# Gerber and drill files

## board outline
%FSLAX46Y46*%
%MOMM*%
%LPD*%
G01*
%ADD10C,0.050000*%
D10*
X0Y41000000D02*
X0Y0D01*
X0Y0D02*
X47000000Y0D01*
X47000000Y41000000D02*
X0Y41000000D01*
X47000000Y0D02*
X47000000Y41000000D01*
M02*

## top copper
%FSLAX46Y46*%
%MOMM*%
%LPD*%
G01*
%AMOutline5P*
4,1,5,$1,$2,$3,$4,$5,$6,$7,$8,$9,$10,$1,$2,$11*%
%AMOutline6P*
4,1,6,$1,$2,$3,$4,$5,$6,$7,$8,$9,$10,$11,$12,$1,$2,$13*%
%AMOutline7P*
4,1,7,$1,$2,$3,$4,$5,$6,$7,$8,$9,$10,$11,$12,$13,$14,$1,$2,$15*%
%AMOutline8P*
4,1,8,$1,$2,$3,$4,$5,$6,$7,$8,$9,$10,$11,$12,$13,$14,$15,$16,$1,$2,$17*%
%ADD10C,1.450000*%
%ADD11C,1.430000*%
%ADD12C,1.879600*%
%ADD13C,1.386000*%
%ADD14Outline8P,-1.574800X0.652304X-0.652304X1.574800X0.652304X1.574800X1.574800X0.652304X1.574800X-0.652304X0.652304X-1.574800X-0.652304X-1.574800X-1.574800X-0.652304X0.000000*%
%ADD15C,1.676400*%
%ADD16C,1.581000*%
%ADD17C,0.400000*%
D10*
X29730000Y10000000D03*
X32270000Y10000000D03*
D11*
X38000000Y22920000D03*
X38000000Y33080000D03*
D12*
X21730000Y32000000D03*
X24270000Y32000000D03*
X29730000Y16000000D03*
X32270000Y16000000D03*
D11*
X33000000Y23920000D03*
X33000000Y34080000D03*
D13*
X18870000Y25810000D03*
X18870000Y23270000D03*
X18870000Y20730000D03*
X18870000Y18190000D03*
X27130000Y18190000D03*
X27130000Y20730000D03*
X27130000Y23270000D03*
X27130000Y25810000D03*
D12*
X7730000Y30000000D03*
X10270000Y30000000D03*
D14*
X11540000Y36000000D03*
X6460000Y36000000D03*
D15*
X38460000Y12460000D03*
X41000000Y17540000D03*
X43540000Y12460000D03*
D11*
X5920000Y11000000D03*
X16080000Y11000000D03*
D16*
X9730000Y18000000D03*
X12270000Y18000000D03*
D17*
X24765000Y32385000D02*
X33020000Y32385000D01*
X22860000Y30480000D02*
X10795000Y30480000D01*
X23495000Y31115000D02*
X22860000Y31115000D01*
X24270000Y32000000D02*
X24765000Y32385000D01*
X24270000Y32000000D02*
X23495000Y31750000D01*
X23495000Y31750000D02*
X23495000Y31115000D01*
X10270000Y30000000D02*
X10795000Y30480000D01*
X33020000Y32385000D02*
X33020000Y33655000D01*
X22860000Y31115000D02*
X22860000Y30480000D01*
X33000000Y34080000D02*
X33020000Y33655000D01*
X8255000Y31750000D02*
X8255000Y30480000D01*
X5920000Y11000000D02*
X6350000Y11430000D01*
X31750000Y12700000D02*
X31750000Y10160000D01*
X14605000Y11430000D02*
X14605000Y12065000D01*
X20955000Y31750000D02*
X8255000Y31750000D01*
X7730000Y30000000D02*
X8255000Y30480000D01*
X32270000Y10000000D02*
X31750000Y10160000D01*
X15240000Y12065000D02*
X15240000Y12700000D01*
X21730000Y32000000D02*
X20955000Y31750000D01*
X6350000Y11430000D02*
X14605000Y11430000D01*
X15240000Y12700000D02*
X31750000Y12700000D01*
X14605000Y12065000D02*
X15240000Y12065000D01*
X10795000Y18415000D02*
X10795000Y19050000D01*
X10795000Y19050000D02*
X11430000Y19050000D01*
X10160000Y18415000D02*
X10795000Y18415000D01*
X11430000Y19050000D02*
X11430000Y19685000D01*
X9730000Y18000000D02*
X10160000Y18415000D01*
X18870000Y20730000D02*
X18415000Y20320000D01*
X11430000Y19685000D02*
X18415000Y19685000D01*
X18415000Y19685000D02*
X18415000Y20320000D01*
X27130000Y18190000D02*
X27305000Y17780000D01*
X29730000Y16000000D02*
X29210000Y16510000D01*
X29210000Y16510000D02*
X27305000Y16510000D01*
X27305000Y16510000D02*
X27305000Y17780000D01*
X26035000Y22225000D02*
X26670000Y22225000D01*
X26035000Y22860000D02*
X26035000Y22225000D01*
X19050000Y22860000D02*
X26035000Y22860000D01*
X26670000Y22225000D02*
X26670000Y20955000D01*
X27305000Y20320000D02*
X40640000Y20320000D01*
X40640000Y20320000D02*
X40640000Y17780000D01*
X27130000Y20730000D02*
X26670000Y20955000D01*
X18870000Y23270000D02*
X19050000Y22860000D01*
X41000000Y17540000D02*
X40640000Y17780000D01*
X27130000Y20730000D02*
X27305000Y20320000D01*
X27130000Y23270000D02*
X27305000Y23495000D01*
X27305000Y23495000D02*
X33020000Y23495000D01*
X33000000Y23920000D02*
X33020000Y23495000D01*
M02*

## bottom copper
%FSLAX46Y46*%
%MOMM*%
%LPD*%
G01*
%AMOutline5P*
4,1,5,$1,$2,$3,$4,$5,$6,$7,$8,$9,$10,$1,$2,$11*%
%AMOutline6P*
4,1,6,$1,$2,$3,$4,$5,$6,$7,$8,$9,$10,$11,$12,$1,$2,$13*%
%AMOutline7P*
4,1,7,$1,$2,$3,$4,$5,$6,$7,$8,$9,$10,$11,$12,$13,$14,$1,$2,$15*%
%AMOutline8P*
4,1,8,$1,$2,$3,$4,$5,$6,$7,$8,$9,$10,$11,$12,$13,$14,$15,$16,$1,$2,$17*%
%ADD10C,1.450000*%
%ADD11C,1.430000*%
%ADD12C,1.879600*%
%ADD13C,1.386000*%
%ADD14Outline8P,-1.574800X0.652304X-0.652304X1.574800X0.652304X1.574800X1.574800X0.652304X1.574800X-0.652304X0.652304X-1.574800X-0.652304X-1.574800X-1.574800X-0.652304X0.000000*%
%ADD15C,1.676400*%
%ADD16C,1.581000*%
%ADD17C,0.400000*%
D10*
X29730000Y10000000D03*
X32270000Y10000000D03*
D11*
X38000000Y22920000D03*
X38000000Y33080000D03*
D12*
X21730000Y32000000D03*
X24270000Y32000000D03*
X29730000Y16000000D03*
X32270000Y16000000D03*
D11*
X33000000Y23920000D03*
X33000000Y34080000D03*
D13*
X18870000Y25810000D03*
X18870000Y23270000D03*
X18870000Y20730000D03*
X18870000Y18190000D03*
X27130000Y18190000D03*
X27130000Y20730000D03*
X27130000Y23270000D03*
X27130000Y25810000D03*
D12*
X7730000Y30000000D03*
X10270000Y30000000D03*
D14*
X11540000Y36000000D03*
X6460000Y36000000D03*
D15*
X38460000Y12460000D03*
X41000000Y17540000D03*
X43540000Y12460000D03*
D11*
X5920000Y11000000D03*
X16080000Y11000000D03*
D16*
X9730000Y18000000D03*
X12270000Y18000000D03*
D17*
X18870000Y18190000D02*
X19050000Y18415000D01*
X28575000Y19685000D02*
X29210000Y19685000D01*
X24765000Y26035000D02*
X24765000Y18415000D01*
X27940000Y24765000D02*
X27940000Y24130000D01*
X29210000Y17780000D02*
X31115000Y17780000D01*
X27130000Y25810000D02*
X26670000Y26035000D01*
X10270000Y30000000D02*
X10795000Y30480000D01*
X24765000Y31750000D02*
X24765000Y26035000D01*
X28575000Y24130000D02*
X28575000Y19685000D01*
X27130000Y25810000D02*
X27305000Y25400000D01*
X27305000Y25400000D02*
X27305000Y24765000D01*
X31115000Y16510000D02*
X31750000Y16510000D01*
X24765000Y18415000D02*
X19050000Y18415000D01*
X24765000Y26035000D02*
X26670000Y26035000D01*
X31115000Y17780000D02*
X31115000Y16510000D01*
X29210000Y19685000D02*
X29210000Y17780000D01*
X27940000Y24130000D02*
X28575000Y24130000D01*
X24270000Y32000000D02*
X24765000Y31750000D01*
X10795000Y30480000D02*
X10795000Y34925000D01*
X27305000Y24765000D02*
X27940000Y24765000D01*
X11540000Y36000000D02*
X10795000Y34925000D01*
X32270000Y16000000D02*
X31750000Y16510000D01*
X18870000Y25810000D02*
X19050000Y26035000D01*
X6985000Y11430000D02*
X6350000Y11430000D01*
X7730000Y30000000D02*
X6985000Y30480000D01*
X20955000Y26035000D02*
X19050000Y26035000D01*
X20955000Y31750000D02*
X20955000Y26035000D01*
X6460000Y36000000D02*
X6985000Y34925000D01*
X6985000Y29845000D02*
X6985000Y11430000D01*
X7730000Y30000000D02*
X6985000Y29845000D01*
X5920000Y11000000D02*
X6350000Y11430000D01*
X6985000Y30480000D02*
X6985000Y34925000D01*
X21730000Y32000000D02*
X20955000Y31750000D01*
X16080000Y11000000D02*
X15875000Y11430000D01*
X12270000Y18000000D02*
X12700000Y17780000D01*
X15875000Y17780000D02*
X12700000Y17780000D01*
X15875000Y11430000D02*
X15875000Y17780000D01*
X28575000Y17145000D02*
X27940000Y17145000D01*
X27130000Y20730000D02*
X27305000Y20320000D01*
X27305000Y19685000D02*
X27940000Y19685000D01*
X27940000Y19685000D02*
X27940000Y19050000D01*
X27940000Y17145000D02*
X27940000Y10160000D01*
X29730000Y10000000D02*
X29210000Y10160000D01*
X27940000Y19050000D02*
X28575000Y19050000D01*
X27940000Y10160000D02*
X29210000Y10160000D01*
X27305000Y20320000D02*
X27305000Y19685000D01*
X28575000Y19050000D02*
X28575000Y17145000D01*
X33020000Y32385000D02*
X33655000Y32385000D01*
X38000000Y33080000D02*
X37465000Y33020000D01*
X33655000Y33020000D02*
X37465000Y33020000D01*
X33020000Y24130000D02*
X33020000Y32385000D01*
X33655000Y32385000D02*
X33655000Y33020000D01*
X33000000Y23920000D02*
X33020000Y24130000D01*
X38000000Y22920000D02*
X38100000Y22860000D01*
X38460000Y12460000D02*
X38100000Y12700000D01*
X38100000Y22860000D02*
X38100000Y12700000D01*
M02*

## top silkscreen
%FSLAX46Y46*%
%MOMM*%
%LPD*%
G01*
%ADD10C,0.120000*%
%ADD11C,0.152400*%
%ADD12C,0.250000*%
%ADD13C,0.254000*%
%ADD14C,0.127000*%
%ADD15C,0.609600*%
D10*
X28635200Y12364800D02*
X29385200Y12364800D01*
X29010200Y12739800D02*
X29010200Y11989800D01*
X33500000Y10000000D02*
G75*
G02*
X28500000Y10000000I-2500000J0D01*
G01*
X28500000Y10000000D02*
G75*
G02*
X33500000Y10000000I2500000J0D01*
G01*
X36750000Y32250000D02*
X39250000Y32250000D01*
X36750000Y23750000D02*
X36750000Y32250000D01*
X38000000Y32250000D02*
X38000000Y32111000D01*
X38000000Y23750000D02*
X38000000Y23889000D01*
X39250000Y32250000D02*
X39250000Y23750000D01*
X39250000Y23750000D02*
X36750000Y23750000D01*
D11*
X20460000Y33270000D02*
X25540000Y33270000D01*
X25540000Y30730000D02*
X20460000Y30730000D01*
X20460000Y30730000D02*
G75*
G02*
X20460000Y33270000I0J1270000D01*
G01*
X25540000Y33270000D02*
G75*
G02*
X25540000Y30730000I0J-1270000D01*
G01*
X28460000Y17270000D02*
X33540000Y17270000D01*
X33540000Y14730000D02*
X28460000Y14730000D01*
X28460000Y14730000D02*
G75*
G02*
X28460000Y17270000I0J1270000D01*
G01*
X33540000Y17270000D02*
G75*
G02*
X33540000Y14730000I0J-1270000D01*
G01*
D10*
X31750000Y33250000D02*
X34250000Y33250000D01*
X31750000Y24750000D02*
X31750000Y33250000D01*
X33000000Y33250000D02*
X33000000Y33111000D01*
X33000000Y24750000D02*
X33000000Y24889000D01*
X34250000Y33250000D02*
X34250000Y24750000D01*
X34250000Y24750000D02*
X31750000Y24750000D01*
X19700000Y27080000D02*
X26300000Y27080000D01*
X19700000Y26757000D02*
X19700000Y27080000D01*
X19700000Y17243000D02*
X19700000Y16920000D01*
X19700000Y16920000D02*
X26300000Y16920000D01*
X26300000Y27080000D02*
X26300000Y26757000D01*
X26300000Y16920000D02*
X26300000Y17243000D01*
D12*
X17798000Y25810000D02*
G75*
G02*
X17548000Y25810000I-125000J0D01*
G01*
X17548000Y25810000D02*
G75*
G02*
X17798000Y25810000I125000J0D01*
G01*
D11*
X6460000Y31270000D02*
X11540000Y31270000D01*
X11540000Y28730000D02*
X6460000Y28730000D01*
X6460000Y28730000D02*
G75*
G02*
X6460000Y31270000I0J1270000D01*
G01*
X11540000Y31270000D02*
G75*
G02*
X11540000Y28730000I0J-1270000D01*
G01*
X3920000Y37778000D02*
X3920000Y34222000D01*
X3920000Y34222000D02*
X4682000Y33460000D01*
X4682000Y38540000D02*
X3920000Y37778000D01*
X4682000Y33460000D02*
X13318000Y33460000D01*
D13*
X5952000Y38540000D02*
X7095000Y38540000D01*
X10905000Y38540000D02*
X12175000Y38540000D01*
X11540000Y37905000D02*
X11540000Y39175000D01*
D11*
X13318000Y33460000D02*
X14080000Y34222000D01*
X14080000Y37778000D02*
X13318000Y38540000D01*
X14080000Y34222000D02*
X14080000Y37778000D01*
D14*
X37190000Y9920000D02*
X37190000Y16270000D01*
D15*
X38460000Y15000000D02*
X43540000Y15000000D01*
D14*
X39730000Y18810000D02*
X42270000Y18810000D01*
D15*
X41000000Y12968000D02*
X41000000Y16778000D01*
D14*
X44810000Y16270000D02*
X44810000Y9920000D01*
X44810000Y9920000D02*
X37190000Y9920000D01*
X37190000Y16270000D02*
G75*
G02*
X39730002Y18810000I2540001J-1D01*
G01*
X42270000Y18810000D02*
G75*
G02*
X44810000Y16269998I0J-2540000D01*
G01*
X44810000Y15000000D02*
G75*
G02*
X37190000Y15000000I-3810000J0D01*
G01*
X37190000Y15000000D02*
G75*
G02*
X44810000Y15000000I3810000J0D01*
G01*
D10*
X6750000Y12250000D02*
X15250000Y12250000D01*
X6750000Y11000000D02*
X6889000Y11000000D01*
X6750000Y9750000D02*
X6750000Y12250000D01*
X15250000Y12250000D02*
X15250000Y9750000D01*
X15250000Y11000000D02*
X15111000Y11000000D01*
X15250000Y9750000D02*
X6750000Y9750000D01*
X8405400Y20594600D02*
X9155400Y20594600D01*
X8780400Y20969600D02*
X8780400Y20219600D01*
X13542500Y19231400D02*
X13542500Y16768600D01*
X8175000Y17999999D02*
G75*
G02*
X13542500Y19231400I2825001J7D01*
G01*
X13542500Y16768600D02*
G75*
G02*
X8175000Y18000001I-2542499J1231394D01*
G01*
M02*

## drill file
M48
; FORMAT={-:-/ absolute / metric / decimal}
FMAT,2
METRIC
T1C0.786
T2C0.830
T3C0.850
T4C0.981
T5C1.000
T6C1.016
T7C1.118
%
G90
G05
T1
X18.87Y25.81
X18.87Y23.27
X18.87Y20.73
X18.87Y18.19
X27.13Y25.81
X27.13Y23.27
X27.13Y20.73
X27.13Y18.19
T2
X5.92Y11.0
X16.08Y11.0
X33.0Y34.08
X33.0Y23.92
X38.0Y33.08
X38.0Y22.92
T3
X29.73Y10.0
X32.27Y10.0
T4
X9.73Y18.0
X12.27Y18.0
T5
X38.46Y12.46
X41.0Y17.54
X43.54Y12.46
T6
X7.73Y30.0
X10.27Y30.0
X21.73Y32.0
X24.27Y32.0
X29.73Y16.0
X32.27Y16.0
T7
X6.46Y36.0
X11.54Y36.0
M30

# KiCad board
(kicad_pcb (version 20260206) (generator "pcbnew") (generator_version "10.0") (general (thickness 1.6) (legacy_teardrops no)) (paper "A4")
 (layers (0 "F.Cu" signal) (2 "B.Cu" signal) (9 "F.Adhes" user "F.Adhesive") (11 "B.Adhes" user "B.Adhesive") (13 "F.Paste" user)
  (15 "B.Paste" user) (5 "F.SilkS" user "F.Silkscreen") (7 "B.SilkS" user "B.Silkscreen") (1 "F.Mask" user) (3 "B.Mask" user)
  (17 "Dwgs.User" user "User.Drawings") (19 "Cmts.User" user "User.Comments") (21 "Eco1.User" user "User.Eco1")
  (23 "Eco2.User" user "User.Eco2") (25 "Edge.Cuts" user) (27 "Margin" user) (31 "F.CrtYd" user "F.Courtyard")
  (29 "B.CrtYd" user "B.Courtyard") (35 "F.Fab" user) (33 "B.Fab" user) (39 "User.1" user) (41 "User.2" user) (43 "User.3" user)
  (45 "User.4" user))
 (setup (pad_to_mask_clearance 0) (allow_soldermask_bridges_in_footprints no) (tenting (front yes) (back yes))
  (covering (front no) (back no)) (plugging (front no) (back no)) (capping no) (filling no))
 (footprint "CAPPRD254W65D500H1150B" (layer "F.Cu") (at 31 -10)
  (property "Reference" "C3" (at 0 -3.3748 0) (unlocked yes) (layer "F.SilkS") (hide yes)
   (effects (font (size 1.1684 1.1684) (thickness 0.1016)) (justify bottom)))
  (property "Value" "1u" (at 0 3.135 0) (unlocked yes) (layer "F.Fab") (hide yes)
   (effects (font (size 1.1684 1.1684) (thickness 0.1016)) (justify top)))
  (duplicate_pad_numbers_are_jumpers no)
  (fp_line (start -2.3648 -2.3648) (end -1.6148 -2.3648) (stroke (width 0.12) (type solid)) (layer "F.SilkS"))
  (fp_line (start -1.9898 -2.7398) (end -1.9898 -1.9898) (stroke (width 0.12) (type solid)) (layer "F.SilkS"))
  (fp_circle (center 0 0) (end 2.5 0) (stroke (width 0.12) (type solid)) (fill no) (layer "F.SilkS"))
  (pad "1" thru_hole circle (at -1.27 0) (size 1.45 1.45) (drill 0.85) (layers "*.Cu" "*.Mask") (remove_unused_layers no) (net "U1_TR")
   (solder_mask_margin 0.1016) (thermal_bridge_angle 0))
  (pad "2" thru_hole circle (at 1.27 0) (size 1.45 1.45) (drill 0.85) (layers "*.Cu" "*.Mask") (remove_unused_layers no) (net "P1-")
   (solder_mask_margin 0.1016) (thermal_bridge_angle 0)))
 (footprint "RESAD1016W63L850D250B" (layer "F.Cu") (at 38 -28 90)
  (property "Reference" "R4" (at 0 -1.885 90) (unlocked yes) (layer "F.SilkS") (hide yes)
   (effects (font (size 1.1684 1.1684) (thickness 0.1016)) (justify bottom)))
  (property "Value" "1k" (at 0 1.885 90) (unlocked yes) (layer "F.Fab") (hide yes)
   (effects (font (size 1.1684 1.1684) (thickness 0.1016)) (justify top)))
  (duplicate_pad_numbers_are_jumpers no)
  (fp_line (start 4.25 -1.25) (end 4.25 1.25) (stroke (width 0.12) (type solid)) (layer "F.SilkS"))
  (fp_line (start -4.25 -1.25) (end 4.25 -1.25) (stroke (width 0.12) (type solid)) (layer "F.SilkS"))
  (fp_line (start 4.25 0) (end 4.111 0) (stroke (width 0.12) (type solid)) (layer "F.SilkS"))
  (fp_line (start -4.25 0) (end -4.111 0) (stroke (width 0.12) (type solid)) (layer "F.SilkS"))
  (fp_line (start 4.25 1.25) (end -4.25 1.25) (stroke (width 0.12) (type solid)) (layer "F.SilkS"))
  (fp_line (start -4.25 1.25) (end -4.25 -1.25) (stroke (width 0.12) (type solid)) (layer "F.SilkS"))
  (pad "1" thru_hole circle (at -5.08 0 90) (size 1.43 1.43) (drill 0.83) (layers "*.Cu" "*.Mask") (remove_unused_layers no)
   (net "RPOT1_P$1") (solder_mask_margin 0.1016) (thermal_bridge_angle 0))
  (pad "2" thru_hole circle (at 5.08 0 90) (size 1.43 1.43) (drill 0.83) (layers "*.Cu" "*.Mask") (remove_unused_layers no) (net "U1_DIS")
   (solder_mask_margin 0.1016) (thermal_bridge_angle 0)))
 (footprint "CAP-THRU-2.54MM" (layer "F.Cu") (at 23 -32)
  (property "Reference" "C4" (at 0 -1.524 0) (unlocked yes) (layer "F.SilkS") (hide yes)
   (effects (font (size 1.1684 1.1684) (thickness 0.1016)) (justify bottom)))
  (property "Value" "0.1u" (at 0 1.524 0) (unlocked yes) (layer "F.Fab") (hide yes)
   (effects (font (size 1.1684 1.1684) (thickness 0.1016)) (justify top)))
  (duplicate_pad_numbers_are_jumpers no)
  (fp_line (start -2.54 -1.27) (end 2.54 -1.27) (stroke (width 0.1524) (type solid)) (layer "F.SilkS"))
  (fp_line (start 2.54 1.27) (end -2.54 1.27) (stroke (width 0.1524) (type solid)) (layer "F.SilkS"))
  (fp_arc (start -2.54 1.27) (mid -3.81 0) (end -2.54 -1.27) (stroke (width 0.1524) (type solid)) (layer "F.SilkS"))
  (fp_arc (start 2.54 -1.27) (mid 3.81 0) (end 2.54 1.27) (stroke (width 0.1524) (type solid)) (layer "F.SilkS"))
  (pad "1" thru_hole circle (at -1.27 0) (size 1.8796 1.8796) (drill 1.016) (layers "*.Cu" "*.Mask") (remove_unused_layers no) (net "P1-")
   (solder_mask_margin 0.1016) (thermal_bridge_angle 0))
  (pad "2" thru_hole circle (at 1.27 0) (size 1.8796 1.8796) (drill 1.016) (layers "*.Cu" "*.Mask") (remove_unused_layers no) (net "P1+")
   (solder_mask_margin 0.1016) (thermal_bridge_angle 0)))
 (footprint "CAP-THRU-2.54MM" (layer "F.Cu") (at 31 -16)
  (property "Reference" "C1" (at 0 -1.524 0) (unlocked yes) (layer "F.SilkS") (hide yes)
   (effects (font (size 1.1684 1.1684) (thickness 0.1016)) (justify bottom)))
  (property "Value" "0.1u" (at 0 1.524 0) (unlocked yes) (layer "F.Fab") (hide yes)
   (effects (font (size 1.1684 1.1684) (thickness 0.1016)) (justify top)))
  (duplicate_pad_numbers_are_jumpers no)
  (fp_line (start -2.54 -1.27) (end 2.54 -1.27) (stroke (width 0.1524) (type solid)) (layer "F.SilkS"))
  (fp_line (start 2.54 1.27) (end -2.54 1.27) (stroke (width 0.1524) (type solid)) (layer "F.SilkS"))
  (fp_arc (start -2.54 1.27) (mid -3.81 0) (end -2.54 -1.27) (stroke (width 0.1524) (type solid)) (layer "F.SilkS"))
  (fp_arc (start 2.54 -1.27) (mid 3.81 0) (end 2.54 1.27) (stroke (width 0.1524) (type solid)) (layer "F.SilkS"))
  (pad "1" thru_hole circle (at -1.27 0) (size 1.8796 1.8796) (drill 1.016) (layers "*.Cu" "*.Mask") (remove_unused_layers no) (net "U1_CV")
   (solder_mask_margin 0.1016) (thermal_bridge_angle 0))
  (pad "2" thru_hole circle (at 1.27 0) (size 1.8796 1.8796) (drill 1.016) (layers "*.Cu" "*.Mask") (remove_unused_layers no) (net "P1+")
   (solder_mask_margin 0.1016) (thermal_bridge_angle 0)))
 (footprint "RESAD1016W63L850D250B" (layer "F.Cu") (at 33 -29 90)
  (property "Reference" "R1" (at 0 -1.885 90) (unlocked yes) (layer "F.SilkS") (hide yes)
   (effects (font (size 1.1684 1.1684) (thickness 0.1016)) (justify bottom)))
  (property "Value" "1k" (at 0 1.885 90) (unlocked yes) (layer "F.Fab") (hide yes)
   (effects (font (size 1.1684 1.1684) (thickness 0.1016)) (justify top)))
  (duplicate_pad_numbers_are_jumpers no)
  (fp_line (start 4.25 -1.25) (end 4.25 1.25) (stroke (width 0.12) (type solid)) (layer "F.SilkS"))
  (fp_line (start -4.25 -1.25) (end 4.25 -1.25) (stroke (width 0.12) (type solid)) (layer "F.SilkS"))
  (fp_line (start 4.25 0) (end 4.111 0) (stroke (width 0.12) (type solid)) (layer "F.SilkS"))
  (fp_line (start -4.25 0) (end -4.111 0) (stroke (width 0.12) (type solid)) (layer "F.SilkS"))
  (fp_line (start 4.25 1.25) (end -4.25 1.25) (stroke (width 0.12) (type solid)) (layer "F.SilkS"))
  (fp_line (start -4.25 1.25) (end -4.25 -1.25) (stroke (width 0.12) (type solid)) (layer "F.SilkS"))
  (pad "1" thru_hole circle (at -5.08 0 90) (size 1.43 1.43) (drill 0.83) (layers "*.Cu" "*.Mask") (remove_unused_layers no) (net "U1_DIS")
   (solder_mask_margin 0.1016) (thermal_bridge_angle 0))
  (pad "2" thru_hole circle (at 5.08 0 90) (size 1.43 1.43) (drill 0.83) (layers "*.Cu" "*.Mask") (remove_unused_layers no) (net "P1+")
   (solder_mask_margin 0.1016) (thermal_bridge_angle 0)))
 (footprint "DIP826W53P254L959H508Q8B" (layer "F.Cu") (at 23 -22)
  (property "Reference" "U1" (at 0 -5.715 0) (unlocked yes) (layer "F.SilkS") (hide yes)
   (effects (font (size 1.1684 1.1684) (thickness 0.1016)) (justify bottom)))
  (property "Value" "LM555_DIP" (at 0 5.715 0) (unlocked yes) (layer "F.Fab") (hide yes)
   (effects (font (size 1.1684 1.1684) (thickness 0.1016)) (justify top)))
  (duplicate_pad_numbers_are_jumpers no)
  (fp_line (start -3.3 -5.08) (end 3.3 -5.08) (stroke (width 0.12) (type solid)) (layer "F.SilkS"))
  (fp_line (start -3.3 -4.757) (end -3.3 -5.08) (stroke (width 0.12) (type solid)) (layer "F.SilkS"))
  (fp_line (start -3.3 4.757) (end -3.3 5.08) (stroke (width 0.12) (type solid)) (layer "F.SilkS"))
  (fp_line (start -3.3 5.08) (end 3.3 5.08) (stroke (width 0.12) (type solid)) (layer "F.SilkS"))
  (fp_line (start 3.3 -5.08) (end 3.3 -4.757) (stroke (width 0.12) (type solid)) (layer "F.SilkS"))
  (fp_line (start 3.3 5.08) (end 3.3 4.757) (stroke (width 0.12) (type solid)) (layer "F.SilkS"))
  (fp_circle (center -5.327 -3.81) (end -5.202 -3.81) (stroke (width 0.25) (type solid)) (fill yes) (layer "F.SilkS"))
  (pad "1" thru_hole circle (at -4.13 -3.81) (size 1.386 1.386) (drill 0.786) (layers "*.Cu" "*.Mask") (remove_unused_layers no) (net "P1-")
   (solder_mask_margin 0.1016) (thermal_bridge_angle 0))
  (pad "2" thru_hole circle (at -4.13 -1.27) (size 1.386 1.386) (drill 0.786) (layers "*.Cu" "*.Mask") (remove_unused_layers no)
   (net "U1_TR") (solder_mask_margin 0.1016) (thermal_bridge_angle 0))
  (pad "3" thru_hole circle (at -4.13 1.27) (size 1.386 1.386) (drill 0.786) (layers "*.Cu" "*.Mask") (remove_unused_layers no)
   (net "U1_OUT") (solder_mask_margin 0.1016) (thermal_bridge_angle 0))
  (pad "4" thru_hole circle (at -4.13 3.81) (size 1.386 1.386) (drill 0.786) (layers "*.Cu" "*.Mask") (remove_unused_layers no) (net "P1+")
   (solder_mask_margin 0.1016) (thermal_bridge_angle 0))
  (pad "5" thru_hole circle (at 4.13 3.81) (size 1.386 1.386) (drill 0.786) (layers "*.Cu" "*.Mask") (remove_unused_layers no) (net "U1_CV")
   (solder_mask_margin 0.1016) (thermal_bridge_angle 0))
  (pad "6" thru_hole circle (at 4.13 1.27) (size 1.386 1.386) (drill 0.786) (layers "*.Cu" "*.Mask") (remove_unused_layers no) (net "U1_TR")
   (solder_mask_margin 0.1016) (thermal_bridge_angle 0))
  (pad "7" thru_hole circle (at 4.13 -1.27) (size 1.386 1.386) (drill 0.786) (layers "*.Cu" "*.Mask") (remove_unused_layers no)
   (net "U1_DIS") (solder_mask_margin 0.1016) (thermal_bridge_angle 0))
  (pad "8" thru_hole circle (at 4.13 -3.81) (size 1.386 1.386) (drill 0.786) (layers "*.Cu" "*.Mask") (remove_unused_layers no) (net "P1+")
   (solder_mask_margin 0.1016) (thermal_bridge_angle 0)))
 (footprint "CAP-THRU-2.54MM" (layer "F.Cu") (at 9 -30)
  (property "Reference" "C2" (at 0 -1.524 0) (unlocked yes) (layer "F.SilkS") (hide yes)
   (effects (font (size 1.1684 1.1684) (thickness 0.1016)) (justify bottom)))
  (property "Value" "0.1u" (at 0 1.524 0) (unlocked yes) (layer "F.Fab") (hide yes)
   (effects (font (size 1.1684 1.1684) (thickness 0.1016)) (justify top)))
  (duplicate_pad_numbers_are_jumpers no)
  (fp_line (start -2.54 -1.27) (end 2.54 -1.27) (stroke (width 0.1524) (type solid)) (layer "F.SilkS"))
  (fp_line (start 2.54 1.27) (end -2.54 1.27) (stroke (width 0.1524) (type solid)) (layer "F.SilkS"))
  (fp_arc (start -2.54 1.27) (mid -3.81 0) (end -2.54 -1.27) (stroke (width 0.1524) (type solid)) (layer "F.SilkS"))
  (fp_arc (start 2.54 -1.27) (mid 3.81 0) (end 2.54 1.27) (stroke (width 0.1524) (type solid)) (layer "F.SilkS"))
  (pad "1" thru_hole circle (at -1.27 0) (size 1.8796 1.8796) (drill 1.016) (layers "*.Cu" "*.Mask") (remove_unused_layers no) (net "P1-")
   (solder_mask_margin 0.1016) (thermal_bridge_angle 0))
  (pad "2" thru_hole circle (at 1.27 0) (size 1.8796 1.8796) (drill 1.016) (layers "*.Cu" "*.Mask") (remove_unused_layers no) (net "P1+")
   (solder_mask_margin 0.1016) (thermal_bridge_angle 0)))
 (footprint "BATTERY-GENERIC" (layer "F.Cu") (at 9 -36)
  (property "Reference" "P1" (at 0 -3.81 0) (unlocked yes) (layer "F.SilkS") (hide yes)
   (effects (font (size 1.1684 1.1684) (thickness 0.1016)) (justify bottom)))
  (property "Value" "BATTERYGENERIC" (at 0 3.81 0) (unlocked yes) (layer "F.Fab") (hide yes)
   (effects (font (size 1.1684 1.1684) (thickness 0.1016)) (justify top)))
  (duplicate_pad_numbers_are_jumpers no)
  (fp_line (start -5.08 -1.778) (end -5.08 1.778) (stroke (width 0.1524) (type solid)) (layer "F.SilkS"))
  (fp_line (start -5.08 1.778) (end -4.318 2.54) (stroke (width 0.1524) (type solid)) (layer "F.SilkS"))
  (fp_line (start -4.318 -2.54) (end -5.08 -1.778) (stroke (width 0.1524) (type solid)) (layer "F.SilkS"))
  (fp_line (start -4.318 2.54) (end 4.318 2.54) (stroke (width 0.1524) (type solid)) (layer "F.SilkS"))
  (fp_line (start -3.048 -2.54) (end -1.905 -2.54) (stroke (width 0.254) (type solid)) (layer "F.SilkS"))
  (fp_line (start 1.905 -2.54) (end 3.175 -2.54) (stroke (width 0.254) (type solid)) (layer "F.SilkS"))
  (fp_line (start 2.54 -1.905) (end 2.54 -3.175) (stroke (width 0.254) (type solid)) (layer "F.SilkS"))
  (fp_line (start 4.318 2.54) (end 5.08 1.778) (stroke (width 0.1524) (type solid)) (layer "F.SilkS"))
  (fp_line (start 5.08 -1.778) (end 4.318 -2.54) (stroke (width 0.1524) (type solid)) (layer "F.SilkS"))
  (fp_line (start 5.08 1.778) (end 5.08 -1.778) (stroke (width 0.1524) (type solid)) (layer "F.SilkS"))
  (pad "+" thru_hole roundrect (at 2.54 0) (size 3.1496 3.1496) (drill 1.1176) (layers "*.Cu" "*.Mask") (remove_unused_layers no)
   (roundrect_rratio 0.25) (chamfer_ratio 0.2928932188) (chamfer top_left top_right bottom_left bottom_right) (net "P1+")
   (solder_mask_margin 0.1016) (thermal_bridge_angle 0))
  (pad "-" thru_hole roundrect (at -2.54 0) (size 3.1496 3.1496) (drill 1.1176) (layers "*.Cu" "*.Mask") (remove_unused_layers no)
   (roundrect_rratio 0.25) (chamfer_ratio 0.2928932188) (chamfer top_left top_right bottom_left bottom_right) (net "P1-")
   (solder_mask_margin 0.1016) (thermal_bridge_angle 0)))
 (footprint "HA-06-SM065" (layer "F.Cu") (at 41 -15)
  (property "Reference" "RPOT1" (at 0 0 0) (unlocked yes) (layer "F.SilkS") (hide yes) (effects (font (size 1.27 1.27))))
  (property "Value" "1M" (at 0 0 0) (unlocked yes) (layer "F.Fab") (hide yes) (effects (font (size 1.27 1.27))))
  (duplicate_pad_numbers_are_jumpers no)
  (fp_line (start -3.81 5.08) (end -3.81 -1.27) (stroke (width 0.127) (type solid)) (layer "F.SilkS"))
  (fp_line (start -2.54 0) (end 2.54 0) (stroke (width 0.6096) (type solid)) (layer "F.SilkS"))
  (fp_line (start -1.27 -3.81) (end 1.27 -3.81) (stroke (width 0.127) (type solid)) (layer "F.SilkS"))
  (fp_line (start 0 2.032) (end 0 -1.778) (stroke (width 0.6096) (type solid)) (layer "F.SilkS"))
  (fp_line (start 3.81 -1.27) (end 3.81 5.08) (stroke (width 0.127) (type solid)) (layer "F.SilkS"))
  (fp_line (start 3.81 5.08) (end -3.81 5.08) (stroke (width 0.127) (type solid)) (layer "F.SilkS"))
  (fp_arc (start -3.81 -1.27) (mid -3.06605 -3.066052) (end -1.269998 -3.81) (stroke (width 0.127) (type solid)) (layer "F.SilkS"))
  (fp_arc (start 1.27 -3.81) (mid 3.066052 -3.06605) (end 3.81 -1.269998) (stroke (width 0.127) (type solid)) (layer "F.SilkS"))
  (fp_circle (center 0 0) (end 3.81 0) (stroke (width 0.127) (type solid)) (fill no) (layer "F.SilkS"))
  (pad "1" thru_hole circle (at -2.54 2.54) (size 1.6764 1.6764) (drill 1) (layers "*.Cu" "*.Mask") (remove_unused_layers no)
   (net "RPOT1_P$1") (solder_mask_margin 0.1016) (thermal_bridge_angle 0))
  (pad "2" thru_hole circle (at 0 -2.54) (size 1.6764 1.6764) (drill 1) (layers "*.Cu" "*.Mask") (remove_unused_layers no) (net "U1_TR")
   (solder_mask_margin 0.1016) (thermal_bridge_angle 0))
  (pad "3" thru_hole circle (at 2.54 2.54) (size 1.6764 1.6764) (drill 1) (layers "*.Cu" "*.Mask") (remove_unused_layers no)
   (solder_mask_margin 0.1016) (thermal_bridge_angle 0)))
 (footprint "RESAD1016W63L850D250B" (layer "F.Cu") (at 11 -11)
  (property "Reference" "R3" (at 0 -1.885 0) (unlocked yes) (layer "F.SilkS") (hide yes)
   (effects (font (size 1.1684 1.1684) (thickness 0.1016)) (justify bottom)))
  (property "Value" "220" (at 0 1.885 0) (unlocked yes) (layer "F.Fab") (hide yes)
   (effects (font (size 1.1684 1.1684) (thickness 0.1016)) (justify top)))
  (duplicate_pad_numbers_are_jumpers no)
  (fp_line (start -4.25 -1.25) (end 4.25 -1.25) (stroke (width 0.12) (type solid)) (layer "F.SilkS"))
  (fp_line (start -4.25 0) (end -4.111 0) (stroke (width 0.12) (type solid)) (layer "F.SilkS"))
  (fp_line (start -4.25 1.25) (end -4.25 -1.25) (stroke (width 0.12) (type solid)) (layer "F.SilkS"))
  (fp_line (start 4.25 -1.25) (end 4.25 1.25) (stroke (width 0.12) (type solid)) (layer "F.SilkS"))
  (fp_line (start 4.25 0) (end 4.111 0) (stroke (width 0.12) (type solid)) (layer "F.SilkS"))
  (fp_line (start 4.25 1.25) (end -4.25 1.25) (stroke (width 0.12) (type solid)) (layer "F.SilkS"))
  (pad "1" thru_hole circle (at -5.08 0) (size 1.43 1.43) (drill 0.83) (layers "*.Cu" "*.Mask") (remove_unused_layers no) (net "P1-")
   (solder_mask_margin 0.1016) (thermal_bridge_angle 0))
  (pad "2" thru_hole circle (at 5.08 0) (size 1.43 1.43) (drill 0.83) (layers "*.Cu" "*.Mask") (remove_unused_layers no) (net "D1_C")
   (solder_mask_margin 0.1016) (thermal_bridge_angle 0)))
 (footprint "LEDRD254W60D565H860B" (layer "F.Cu") (at 11 -18)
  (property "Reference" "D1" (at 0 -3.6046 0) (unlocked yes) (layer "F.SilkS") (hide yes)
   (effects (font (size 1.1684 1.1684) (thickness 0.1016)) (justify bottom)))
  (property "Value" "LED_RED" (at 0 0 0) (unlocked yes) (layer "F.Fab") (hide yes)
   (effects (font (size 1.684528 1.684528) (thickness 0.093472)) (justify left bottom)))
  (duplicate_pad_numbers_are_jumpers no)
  (fp_line (start -2.5946 -2.5946) (end -1.8446 -2.5946) (stroke (width 0.12) (type solid)) (layer "F.SilkS"))
  (fp_line (start -2.2196 -2.9696) (end -2.2196 -2.2196) (stroke (width 0.12) (type solid)) (layer "F.SilkS"))
  (fp_line (start 2.5425 -1.2314) (end 2.5425 1.2314) (stroke (width 0.12) (type solid)) (layer "F.SilkS"))
  (fp_arc (start -2.825 0.000001) (mid -0.631694 -2.753475) (end 2.5425 -1.2314) (stroke (width 0.12) (type solid)) (layer "F.SilkS"))
  (fp_arc (start 2.5425 1.2314) (mid -0.631694 2.753475) (end -2.825 -0.000001) (stroke (width 0.12) (type solid)) (layer "F.SilkS"))
  (pad "1" thru_hole circle (at -1.27 0) (size 1.581 1.581) (drill 0.981) (layers "*.Cu" "*.Mask") (remove_unused_layers no) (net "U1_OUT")
   (solder_mask_margin 0.1016) (thermal_bridge_angle 0))
  (pad "2" thru_hole circle (at 1.27 0) (size 1.581 1.581) (drill 0.981) (layers "*.Cu" "*.Mask") (remove_unused_layers no) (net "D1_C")
   (solder_mask_margin 0.1016) (thermal_bridge_angle 0)))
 (gr_line (start 0 -41) (end 0 0) (stroke (width 0.05) (type solid)) (layer "Edge.Cuts"))
 (gr_line (start 0 0) (end 47 0) (stroke (width 0.05) (type solid)) (layer "Edge.Cuts"))
 (gr_line (start 47 -41) (end 0 -41) (stroke (width 0.05) (type solid)) (layer "Edge.Cuts"))
 (gr_line (start 47 0) (end 47 -41) (stroke (width 0.05) (type solid)) (layer "Edge.Cuts"))
 (segment (start 24.765 -32.385) (end 33.02 -32.385) (width 0.4) (layer "F.Cu") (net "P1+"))
 (segment (start 22.86 -30.48) (end 10.795 -30.48) (width 0.4) (layer "F.Cu") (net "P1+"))
 (segment (start 23.495 -31.115) (end 22.86 -31.115) (width 0.4) (layer "F.Cu") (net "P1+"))
 (segment (start 24.27 -32) (end 24.765 -32.385) (width 0.4) (layer "F.Cu") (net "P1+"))
 (segment (start 24.27 -32) (end 23.495 -31.75) (width 0.4) (layer "F.Cu") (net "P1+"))
 (segment (start 23.495 -31.75) (end 23.495 -31.115) (width 0.4) (layer "F.Cu") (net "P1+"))
 (segment (start 10.27 -30) (end 10.795 -30.48) (width 0.4) (layer "F.Cu") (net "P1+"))
 (segment (start 33.02 -32.385) (end 33.02 -33.655) (width 0.4) (layer "F.Cu") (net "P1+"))
 (segment (start 22.86 -31.115) (end 22.86 -30.48) (width 0.4) (layer "F.Cu") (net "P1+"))
 (segment (start 33 -34.08) (end 33.02 -33.655) (width 0.4) (layer "F.Cu") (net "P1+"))
 (segment (start 18.87 -18.19) (end 19.05 -18.415) (width 0.4) (layer "B.Cu") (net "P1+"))
 (segment (start 28.575 -19.685) (end 29.21 -19.685) (width 0.4) (layer "B.Cu") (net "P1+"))
 (segment (start 24.765 -26.035) (end 24.765 -18.415) (width 0.4) (layer "B.Cu") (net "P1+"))
 (segment (start 27.94 -24.765) (end 27.94 -24.13) (width 0.4) (layer "B.Cu") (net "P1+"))
 (segment (start 29.21 -17.78) (end 31.115 -17.78) (width 0.4) (layer "B.Cu") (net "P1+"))
 (segment (start 27.13 -25.81) (end 26.67 -26.035) (width 0.4) (layer "B.Cu") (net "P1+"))
 (segment (start 10.27 -30) (end 10.795 -30.48) (width 0.4) (layer "B.Cu") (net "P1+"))
 (segment (start 24.765 -31.75) (end 24.765 -26.035) (width 0.4) (layer "B.Cu") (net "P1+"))
 (segment (start 28.575 -24.13) (end 28.575 -19.685) (width 0.4) (layer "B.Cu") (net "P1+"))
 (segment (start 27.13 -25.81) (end 27.305 -25.4) (width 0.4) (layer "B.Cu") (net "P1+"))
 (segment (start 27.305 -25.4) (end 27.305 -24.765) (width 0.4) (layer "B.Cu") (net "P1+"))
 (segment (start 31.115 -16.51) (end 31.75 -16.51) (width 0.4) (layer "B.Cu") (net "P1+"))
 (segment (start 24.765 -18.415) (end 19.05 -18.415) (width 0.4) (layer "B.Cu") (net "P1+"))
 (segment (start 24.765 -26.035) (end 26.67 -26.035) (width 0.4) (layer "B.Cu") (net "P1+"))
 (segment (start 31.115 -17.78) (end 31.115 -16.51) (width 0.4) (layer "B.Cu") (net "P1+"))
 (segment (start 29.21 -19.685) (end 29.21 -17.78) (width 0.4) (layer "B.Cu") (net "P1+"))
 (segment (start 27.94 -24.13) (end 28.575 -24.13) (width 0.4) (layer "B.Cu") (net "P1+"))
 (segment (start 24.27 -32) (end 24.765 -31.75) (width 0.4) (layer "B.Cu") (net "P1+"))
 (segment (start 10.795 -30.48) (end 10.795 -34.925) (width 0.4) (layer "B.Cu") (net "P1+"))
 (segment (start 27.305 -24.765) (end 27.94 -24.765) (width 0.4) (layer "B.Cu") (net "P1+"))
 (segment (start 11.54 -36) (end 10.795 -34.925) (width 0.4) (layer "B.Cu") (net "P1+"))
 (segment (start 32.27 -16) (end 31.75 -16.51) (width 0.4) (layer "B.Cu") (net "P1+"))
 (segment (start 8.255 -31.75) (end 8.255 -30.48) (width 0.4) (layer "F.Cu") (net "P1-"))
 (segment (start 5.92 -11) (end 6.35 -11.43) (width 0.4) (layer "F.Cu") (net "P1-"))
 (segment (start 31.75 -12.7) (end 31.75 -10.16) (width 0.4) (layer "F.Cu") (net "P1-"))
 (segment (start 14.605 -11.43) (end 14.605 -12.065) (width 0.4) (layer "F.Cu") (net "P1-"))
 (segment (start 20.955 -31.75) (end 8.255 -31.75) (width 0.4) (layer "F.Cu") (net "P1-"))
 (segment (start 7.73 -30) (end 8.255 -30.48) (width 0.4) (layer "F.Cu") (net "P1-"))
 (segment (start 32.27 -10) (end 31.75 -10.16) (width 0.4) (layer "F.Cu") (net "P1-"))
 (segment (start 15.24 -12.065) (end 15.24 -12.7) (width 0.4) (layer "F.Cu") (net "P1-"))
 (segment (start 21.73 -32) (end 20.955 -31.75) (width 0.4) (layer "F.Cu") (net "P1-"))
 (segment (start 6.35 -11.43) (end 14.605 -11.43) (width 0.4) (layer "F.Cu") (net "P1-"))
 (segment (start 15.24 -12.7) (end 31.75 -12.7) (width 0.4) (layer "F.Cu") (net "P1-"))
 (segment (start 14.605 -12.065) (end 15.24 -12.065) (width 0.4) (layer "F.Cu") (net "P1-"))
 (segment (start 18.87 -25.81) (end 19.05 -26.035) (width 0.4) (layer "B.Cu") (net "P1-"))
 (segment (start 6.985 -11.43) (end 6.35 -11.43) (width 0.4) (layer "B.Cu") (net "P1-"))
 (segment (start 7.73 -30) (end 6.985 -30.48) (width 0.4) (layer "B.Cu") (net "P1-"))
 (segment (start 20.955 -26.035) (end 19.05 -26.035) (width 0.4) (layer "B.Cu") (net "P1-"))
 (segment (start 20.955 -31.75) (end 20.955 -26.035) (width 0.4) (layer "B.Cu") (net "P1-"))
 (segment (start 6.46 -36) (end 6.985 -34.925) (width 0.4) (layer "B.Cu") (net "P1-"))
 (segment (start 6.985 -29.845) (end 6.985 -11.43) (width 0.4) (layer "B.Cu") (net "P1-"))
 (segment (start 7.73 -30) (end 6.985 -29.845) (width 0.4) (layer "B.Cu") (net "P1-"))
 (segment (start 5.92 -11) (end 6.35 -11.43) (width 0.4) (layer "B.Cu") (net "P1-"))
 (segment (start 6.985 -30.48) (end 6.985 -34.925) (width 0.4) (layer "B.Cu") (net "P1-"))
 (segment (start 21.73 -32) (end 20.955 -31.75) (width 0.4) (layer "B.Cu") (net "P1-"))
 (segment (start 16.08 -11) (end 15.875 -11.43) (width 0.4) (layer "B.Cu") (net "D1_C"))
 (segment (start 12.27 -18) (end 12.7 -17.78) (width 0.4) (layer "B.Cu") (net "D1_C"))
 (segment (start 15.875 -17.78) (end 12.7 -17.78) (width 0.4) (layer "B.Cu") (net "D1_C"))
 (segment (start 15.875 -11.43) (end 15.875 -17.78) (width 0.4) (layer "B.Cu") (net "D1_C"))
 (segment (start 10.795 -18.415) (end 10.795 -19.05) (width 0.4) (layer "F.Cu") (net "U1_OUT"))
 (segment (start 10.795 -19.05) (end 11.43 -19.05) (width 0.4) (layer "F.Cu") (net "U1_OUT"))
 (segment (start 10.16 -18.415) (end 10.795 -18.415) (width 0.4) (layer "F.Cu") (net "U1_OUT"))
 (segment (start 11.43 -19.05) (end 11.43 -19.685) (width 0.4) (layer "F.Cu") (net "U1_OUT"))
 (segment (start 9.73 -18) (end 10.16 -18.415) (width 0.4) (layer "F.Cu") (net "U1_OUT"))
 (segment (start 18.87 -20.73) (end 18.415 -20.32) (width 0.4) (layer "F.Cu") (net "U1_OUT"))
 (segment (start 11.43 -19.685) (end 18.415 -19.685) (width 0.4) (layer "F.Cu") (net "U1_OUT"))
 (segment (start 18.415 -19.685) (end 18.415 -20.32) (width 0.4) (layer "F.Cu") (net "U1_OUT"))
 (segment (start 27.13 -18.19) (end 27.305 -17.78) (width 0.4) (layer "F.Cu") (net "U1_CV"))
 (segment (start 29.73 -16) (end 29.21 -16.51) (width 0.4) (layer "F.Cu") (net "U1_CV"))
 (segment (start 29.21 -16.51) (end 27.305 -16.51) (width 0.4) (layer "F.Cu") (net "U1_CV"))
 (segment (start 27.305 -16.51) (end 27.305 -17.78) (width 0.4) (layer "F.Cu") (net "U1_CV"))
 (segment (start 26.035 -22.225) (end 26.67 -22.225) (width 0.4) (layer "F.Cu") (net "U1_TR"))
 (segment (start 26.035 -22.86) (end 26.035 -22.225) (width 0.4) (layer "F.Cu") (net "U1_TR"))
 (segment (start 19.05 -22.86) (end 26.035 -22.86) (width 0.4) (layer "F.Cu") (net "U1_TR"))
 (segment (start 26.67 -22.225) (end 26.67 -20.955) (width 0.4) (layer "F.Cu") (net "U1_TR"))
 (segment (start 27.305 -20.32) (end 40.64 -20.32) (width 0.4) (layer "F.Cu") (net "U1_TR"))
 (segment (start 40.64 -20.32) (end 40.64 -17.78) (width 0.4) (layer "F.Cu") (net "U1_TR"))
 (segment (start 27.13 -20.73) (end 26.67 -20.955) (width 0.4) (layer "F.Cu") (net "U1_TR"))
 (segment (start 18.87 -23.27) (end 19.05 -22.86) (width 0.4) (layer "F.Cu") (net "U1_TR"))
 (segment (start 41 -17.54) (end 40.64 -17.78) (width 0.4) (layer "F.Cu") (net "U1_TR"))
 (segment (start 27.13 -20.73) (end 27.305 -20.32) (width 0.4) (layer "F.Cu") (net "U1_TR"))
 (segment (start 28.575 -17.145) (end 27.94 -17.145) (width 0.4) (layer "B.Cu") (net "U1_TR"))
 (segment (start 27.13 -20.73) (end 27.305 -20.32) (width 0.4) (layer "B.Cu") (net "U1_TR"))
 (segment (start 27.305 -19.685) (end 27.94 -19.685) (width 0.4) (layer "B.Cu") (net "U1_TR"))
 (segment (start 27.94 -19.685) (end 27.94 -19.05) (width 0.4) (layer "B.Cu") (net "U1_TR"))
 (segment (start 27.94 -17.145) (end 27.94 -10.16) (width 0.4) (layer "B.Cu") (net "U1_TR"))
 (segment (start 29.73 -10) (end 29.21 -10.16) (width 0.4) (layer "B.Cu") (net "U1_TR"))
 (segment (start 27.94 -19.05) (end 28.575 -19.05) (width 0.4) (layer "B.Cu") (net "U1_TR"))
 (segment (start 27.94 -10.16) (end 29.21 -10.16) (width 0.4) (layer "B.Cu") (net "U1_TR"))
 (segment (start 27.305 -20.32) (end 27.305 -19.685) (width 0.4) (layer "B.Cu") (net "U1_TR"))
 (segment (start 28.575 -19.05) (end 28.575 -17.145) (width 0.4) (layer "B.Cu") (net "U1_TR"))
 (segment (start 27.13 -23.27) (end 27.305 -23.495) (width 0.4) (layer "F.Cu") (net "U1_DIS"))
 (segment (start 27.305 -23.495) (end 33.02 -23.495) (width 0.4) (layer "F.Cu") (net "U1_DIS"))
 (segment (start 33 -23.92) (end 33.02 -23.495) (width 0.4) (layer "F.Cu") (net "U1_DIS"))
 (segment (start 33.02 -32.385) (end 33.655 -32.385) (width 0.4) (layer "B.Cu") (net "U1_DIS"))
 (segment (start 38 -33.08) (end 37.465 -33.02) (width 0.4) (layer "B.Cu") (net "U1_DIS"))
 (segment (start 33.655 -33.02) (end 37.465 -33.02) (width 0.4) (layer "B.Cu") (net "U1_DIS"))
 (segment (start 33.02 -24.13) (end 33.02 -32.385) (width 0.4) (layer "B.Cu") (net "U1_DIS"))
 (segment (start 33.655 -32.385) (end 33.655 -33.02) (width 0.4) (layer "B.Cu") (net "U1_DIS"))
 (segment (start 33 -23.92) (end 33.02 -24.13) (width 0.4) (layer "B.Cu") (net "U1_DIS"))
 (segment (start 38 -22.92) (end 38.1 -22.86) (width 0.4) (layer "B.Cu") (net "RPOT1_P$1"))
 (segment (start 38.46 -12.46) (end 38.1 -12.7) (width 0.4) (layer "B.Cu") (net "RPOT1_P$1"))
 (segment (start 38.1 -22.86) (end 38.1 -12.7) (width 0.4) (layer "B.Cu") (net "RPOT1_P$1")))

